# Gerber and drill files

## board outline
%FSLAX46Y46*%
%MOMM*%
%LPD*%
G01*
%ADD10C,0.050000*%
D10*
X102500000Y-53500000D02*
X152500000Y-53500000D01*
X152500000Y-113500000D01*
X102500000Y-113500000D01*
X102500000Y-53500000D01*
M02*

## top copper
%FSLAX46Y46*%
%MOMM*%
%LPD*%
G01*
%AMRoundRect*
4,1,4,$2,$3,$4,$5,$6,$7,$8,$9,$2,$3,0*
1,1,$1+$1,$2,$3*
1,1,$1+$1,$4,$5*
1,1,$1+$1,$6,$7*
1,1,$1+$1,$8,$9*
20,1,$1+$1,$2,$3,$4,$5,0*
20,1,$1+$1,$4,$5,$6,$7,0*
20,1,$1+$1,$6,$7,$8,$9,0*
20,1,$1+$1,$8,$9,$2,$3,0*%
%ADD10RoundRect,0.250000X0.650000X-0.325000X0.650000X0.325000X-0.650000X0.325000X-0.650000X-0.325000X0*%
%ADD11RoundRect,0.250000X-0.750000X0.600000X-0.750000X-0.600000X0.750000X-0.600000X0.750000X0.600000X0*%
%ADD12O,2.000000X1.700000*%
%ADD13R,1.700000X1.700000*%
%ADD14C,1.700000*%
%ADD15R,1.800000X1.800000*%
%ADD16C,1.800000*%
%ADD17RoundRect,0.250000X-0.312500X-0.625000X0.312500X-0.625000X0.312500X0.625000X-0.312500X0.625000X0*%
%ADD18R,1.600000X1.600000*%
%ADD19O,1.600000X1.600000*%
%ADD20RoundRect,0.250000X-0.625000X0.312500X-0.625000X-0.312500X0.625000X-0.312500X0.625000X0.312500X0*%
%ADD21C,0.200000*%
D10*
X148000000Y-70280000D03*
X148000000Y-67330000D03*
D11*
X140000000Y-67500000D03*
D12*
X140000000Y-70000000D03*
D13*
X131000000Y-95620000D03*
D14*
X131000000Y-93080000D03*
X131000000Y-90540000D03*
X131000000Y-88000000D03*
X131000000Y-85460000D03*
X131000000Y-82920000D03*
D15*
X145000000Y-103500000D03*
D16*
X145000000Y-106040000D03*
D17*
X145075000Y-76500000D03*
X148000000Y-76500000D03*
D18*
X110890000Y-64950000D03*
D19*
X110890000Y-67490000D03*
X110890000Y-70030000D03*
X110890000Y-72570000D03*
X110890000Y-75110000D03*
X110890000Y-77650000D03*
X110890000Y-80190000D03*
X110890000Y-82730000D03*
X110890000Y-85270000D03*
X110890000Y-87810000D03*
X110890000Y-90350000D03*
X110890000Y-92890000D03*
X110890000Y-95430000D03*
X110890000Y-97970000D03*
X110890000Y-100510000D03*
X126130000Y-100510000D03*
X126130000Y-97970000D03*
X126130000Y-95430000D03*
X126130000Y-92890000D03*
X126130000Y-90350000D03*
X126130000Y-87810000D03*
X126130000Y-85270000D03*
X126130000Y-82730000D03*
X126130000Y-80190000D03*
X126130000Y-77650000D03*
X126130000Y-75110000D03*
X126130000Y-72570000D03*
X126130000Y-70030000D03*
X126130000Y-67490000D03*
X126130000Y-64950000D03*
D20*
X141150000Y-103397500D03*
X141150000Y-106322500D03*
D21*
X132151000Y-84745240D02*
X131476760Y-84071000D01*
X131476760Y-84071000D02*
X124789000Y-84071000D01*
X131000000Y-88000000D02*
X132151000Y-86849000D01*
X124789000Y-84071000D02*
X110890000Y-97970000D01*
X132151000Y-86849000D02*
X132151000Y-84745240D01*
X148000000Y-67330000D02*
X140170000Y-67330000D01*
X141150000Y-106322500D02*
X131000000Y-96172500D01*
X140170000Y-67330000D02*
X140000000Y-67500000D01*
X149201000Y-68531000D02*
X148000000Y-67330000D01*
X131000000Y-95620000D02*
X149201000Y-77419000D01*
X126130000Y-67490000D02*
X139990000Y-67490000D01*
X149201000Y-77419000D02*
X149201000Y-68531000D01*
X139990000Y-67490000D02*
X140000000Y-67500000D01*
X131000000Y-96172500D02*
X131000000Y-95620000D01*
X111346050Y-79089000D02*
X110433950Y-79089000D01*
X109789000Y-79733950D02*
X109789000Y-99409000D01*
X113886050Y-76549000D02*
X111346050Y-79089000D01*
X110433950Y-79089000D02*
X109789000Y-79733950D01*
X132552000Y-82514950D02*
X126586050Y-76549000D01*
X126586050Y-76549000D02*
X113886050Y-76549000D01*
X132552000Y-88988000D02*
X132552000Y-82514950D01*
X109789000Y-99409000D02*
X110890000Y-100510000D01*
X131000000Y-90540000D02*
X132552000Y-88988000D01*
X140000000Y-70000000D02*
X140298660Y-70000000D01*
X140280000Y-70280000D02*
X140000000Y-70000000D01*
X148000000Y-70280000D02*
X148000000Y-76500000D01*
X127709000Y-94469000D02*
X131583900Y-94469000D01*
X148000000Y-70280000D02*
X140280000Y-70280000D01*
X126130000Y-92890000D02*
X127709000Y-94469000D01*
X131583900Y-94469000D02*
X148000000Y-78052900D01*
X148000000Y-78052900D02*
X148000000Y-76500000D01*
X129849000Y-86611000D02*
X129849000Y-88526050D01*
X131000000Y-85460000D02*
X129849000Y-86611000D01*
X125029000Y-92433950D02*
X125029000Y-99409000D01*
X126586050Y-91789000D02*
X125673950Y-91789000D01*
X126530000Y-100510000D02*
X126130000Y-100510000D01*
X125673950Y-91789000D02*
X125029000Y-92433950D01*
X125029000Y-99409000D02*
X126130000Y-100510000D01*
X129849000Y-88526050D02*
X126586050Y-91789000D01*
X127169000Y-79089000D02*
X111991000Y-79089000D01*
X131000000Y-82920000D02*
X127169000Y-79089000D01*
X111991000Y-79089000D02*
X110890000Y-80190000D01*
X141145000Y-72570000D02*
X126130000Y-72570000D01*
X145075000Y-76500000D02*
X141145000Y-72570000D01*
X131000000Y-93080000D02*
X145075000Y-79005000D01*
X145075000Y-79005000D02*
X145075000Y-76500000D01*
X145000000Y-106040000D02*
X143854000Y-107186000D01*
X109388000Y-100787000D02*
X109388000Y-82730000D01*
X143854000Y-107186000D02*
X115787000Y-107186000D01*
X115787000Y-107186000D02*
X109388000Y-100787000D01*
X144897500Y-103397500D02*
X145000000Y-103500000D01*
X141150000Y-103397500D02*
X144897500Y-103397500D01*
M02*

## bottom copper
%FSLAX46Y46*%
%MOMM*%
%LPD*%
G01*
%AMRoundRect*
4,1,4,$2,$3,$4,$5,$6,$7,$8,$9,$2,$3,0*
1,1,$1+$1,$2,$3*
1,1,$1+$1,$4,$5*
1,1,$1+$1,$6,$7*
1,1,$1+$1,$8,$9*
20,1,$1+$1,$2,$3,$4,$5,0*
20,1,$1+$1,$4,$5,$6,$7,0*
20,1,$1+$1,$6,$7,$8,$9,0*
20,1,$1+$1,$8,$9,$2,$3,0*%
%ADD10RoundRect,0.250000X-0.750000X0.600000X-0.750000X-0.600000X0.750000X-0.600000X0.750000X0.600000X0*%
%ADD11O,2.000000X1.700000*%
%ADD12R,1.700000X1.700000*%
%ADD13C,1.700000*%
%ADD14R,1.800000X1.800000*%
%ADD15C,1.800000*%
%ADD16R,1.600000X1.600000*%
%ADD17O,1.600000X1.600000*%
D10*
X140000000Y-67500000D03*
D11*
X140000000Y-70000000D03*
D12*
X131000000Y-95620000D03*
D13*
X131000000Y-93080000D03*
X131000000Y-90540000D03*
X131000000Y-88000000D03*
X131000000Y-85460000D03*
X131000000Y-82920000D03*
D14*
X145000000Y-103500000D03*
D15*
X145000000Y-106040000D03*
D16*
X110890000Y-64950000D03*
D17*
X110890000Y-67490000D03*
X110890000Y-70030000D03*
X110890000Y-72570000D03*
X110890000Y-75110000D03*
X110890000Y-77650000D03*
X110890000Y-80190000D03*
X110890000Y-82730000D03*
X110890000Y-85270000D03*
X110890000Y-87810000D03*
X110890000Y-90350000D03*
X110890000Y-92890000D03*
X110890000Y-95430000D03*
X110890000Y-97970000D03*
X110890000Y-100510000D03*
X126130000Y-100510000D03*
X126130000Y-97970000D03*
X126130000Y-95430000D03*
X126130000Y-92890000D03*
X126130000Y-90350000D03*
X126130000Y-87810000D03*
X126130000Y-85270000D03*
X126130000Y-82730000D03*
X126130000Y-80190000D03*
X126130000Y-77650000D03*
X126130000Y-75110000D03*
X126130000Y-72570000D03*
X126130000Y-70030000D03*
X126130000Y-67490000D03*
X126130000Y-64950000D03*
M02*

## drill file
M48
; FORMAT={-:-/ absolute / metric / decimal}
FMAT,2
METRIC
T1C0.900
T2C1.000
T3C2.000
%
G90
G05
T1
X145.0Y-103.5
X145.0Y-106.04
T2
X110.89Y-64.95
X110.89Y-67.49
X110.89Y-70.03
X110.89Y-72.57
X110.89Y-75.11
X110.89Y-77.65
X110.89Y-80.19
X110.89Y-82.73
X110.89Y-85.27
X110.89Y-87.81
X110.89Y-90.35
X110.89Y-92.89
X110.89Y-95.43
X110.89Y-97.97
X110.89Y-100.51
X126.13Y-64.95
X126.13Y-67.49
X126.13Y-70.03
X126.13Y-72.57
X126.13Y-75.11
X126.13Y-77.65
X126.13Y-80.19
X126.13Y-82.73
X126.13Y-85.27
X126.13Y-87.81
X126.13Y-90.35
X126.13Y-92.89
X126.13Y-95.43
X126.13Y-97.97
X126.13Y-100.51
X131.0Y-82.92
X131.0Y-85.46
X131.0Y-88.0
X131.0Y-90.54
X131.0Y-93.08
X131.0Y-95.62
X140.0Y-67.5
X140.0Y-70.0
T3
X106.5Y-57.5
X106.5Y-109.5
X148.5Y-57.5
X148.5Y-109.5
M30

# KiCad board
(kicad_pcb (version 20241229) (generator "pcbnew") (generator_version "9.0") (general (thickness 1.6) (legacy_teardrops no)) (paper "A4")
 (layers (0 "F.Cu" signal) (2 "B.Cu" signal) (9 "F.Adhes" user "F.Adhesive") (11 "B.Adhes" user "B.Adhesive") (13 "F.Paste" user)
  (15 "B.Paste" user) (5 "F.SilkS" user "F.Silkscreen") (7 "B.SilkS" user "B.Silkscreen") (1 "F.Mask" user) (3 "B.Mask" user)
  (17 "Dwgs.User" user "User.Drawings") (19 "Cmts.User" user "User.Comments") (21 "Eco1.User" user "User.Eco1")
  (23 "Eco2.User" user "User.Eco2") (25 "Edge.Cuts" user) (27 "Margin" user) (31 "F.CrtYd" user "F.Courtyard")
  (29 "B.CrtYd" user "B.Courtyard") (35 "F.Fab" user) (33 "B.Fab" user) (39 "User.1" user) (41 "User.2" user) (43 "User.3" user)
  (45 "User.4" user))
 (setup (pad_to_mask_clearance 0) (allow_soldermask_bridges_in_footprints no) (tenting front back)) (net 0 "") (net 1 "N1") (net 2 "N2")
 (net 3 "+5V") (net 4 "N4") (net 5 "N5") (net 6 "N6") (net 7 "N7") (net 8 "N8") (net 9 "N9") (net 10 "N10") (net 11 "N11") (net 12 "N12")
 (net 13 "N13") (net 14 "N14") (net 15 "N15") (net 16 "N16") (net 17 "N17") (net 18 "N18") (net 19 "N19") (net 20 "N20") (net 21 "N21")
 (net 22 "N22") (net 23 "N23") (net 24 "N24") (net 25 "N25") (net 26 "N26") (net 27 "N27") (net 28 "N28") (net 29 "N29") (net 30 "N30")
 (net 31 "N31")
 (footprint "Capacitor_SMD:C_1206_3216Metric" (layer "F.Cu") (at 148 68.805 90)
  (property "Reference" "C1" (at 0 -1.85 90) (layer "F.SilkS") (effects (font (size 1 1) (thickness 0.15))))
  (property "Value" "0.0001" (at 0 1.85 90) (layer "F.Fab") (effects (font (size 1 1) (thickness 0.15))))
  (pad "1" smd roundrect (at -1.475 0 90) (size 1.15 1.8) (layers "F.Cu" "F.Mask" "F.Paste") (roundrect_rratio 0.217391) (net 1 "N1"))
  (pad "2" smd roundrect (at 1.475 0 90) (size 1.15 1.8) (layers "F.Cu" "F.Mask" "F.Paste") (roundrect_rratio 0.217391) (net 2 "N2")))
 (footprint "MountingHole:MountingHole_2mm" (layer "F.Cu") (at 148.5 57.5)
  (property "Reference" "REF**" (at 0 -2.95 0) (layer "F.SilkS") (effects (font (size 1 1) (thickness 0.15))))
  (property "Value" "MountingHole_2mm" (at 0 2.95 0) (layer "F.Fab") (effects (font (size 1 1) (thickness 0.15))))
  (pad "" np_thru_hole circle (at 0 0) (size 2 2) (drill 2) (layers "*.Cu" "*.Mask")))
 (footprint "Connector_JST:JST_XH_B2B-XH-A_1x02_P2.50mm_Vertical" (layer "F.Cu") (at 140 67.5 -90)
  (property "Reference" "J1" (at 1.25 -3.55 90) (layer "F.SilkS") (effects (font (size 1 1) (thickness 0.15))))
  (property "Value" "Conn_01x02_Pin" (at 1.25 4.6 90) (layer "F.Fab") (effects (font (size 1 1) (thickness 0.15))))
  (pad "1" thru_hole roundrect (at 0 0 270) (size 1.7 2) (drill 1) (layers "*.Cu" "*.Mask") (remove_unused_layers no)
   (roundrect_rratio 0.147059) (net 2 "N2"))
  (pad "2" thru_hole oval (at 2.5 0 270) (size 1.7 2) (drill 1) (layers "*.Cu" "*.Mask") (remove_unused_layers no) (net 1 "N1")))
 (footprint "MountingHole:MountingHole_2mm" (layer "F.Cu") (at 148.5 109.5)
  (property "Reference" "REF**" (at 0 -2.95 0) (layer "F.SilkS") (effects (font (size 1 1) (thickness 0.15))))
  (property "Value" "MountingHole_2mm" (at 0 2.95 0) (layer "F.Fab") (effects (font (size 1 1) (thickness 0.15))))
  (pad "" np_thru_hole circle (at 0 0) (size 2 2) (drill 2) (layers "*.Cu" "*.Mask")))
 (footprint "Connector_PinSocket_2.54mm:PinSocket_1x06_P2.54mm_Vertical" (layer "F.Cu") (at 131 95.62 180)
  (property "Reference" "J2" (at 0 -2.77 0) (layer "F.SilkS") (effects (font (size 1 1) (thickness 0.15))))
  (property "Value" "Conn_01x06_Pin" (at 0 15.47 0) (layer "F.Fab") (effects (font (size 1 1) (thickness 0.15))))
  (pad "1" thru_hole rect (at 0 0 180) (size 1.7 1.7) (drill 1) (layers "*.Cu" "*.Mask") (remove_unused_layers no) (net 2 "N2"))
  (pad "2" thru_hole circle (at 0 2.54 180) (size 1.7 1.7) (drill 1) (layers "*.Cu" "*.Mask") (remove_unused_layers no) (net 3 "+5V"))
  (pad "3" thru_hole circle (at 0 5.08 180) (size 1.7 1.7) (drill 1) (layers "*.Cu" "*.Mask") (remove_unused_layers no) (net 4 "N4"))
  (pad "4" thru_hole circle (at 0 7.62 180) (size 1.7 1.7) (drill 1) (layers "*.Cu" "*.Mask") (remove_unused_layers no) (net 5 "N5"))
  (pad "5" thru_hole circle (at 0 10.16 180) (size 1.7 1.7) (drill 1) (layers "*.Cu" "*.Mask") (remove_unused_layers no) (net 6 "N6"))
  (pad "6" thru_hole circle (at 0 12.7 180) (size 1.7 1.7) (drill 1) (layers "*.Cu" "*.Mask") (remove_unused_layers no) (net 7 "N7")))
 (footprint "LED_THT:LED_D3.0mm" (layer "F.Cu") (at 145 103.5 -90)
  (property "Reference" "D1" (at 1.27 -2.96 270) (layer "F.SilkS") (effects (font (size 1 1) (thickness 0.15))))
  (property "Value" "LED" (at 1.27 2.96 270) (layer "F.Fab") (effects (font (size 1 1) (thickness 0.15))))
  (pad "1" thru_hole rect (at 0 0 270) (size 1.8 1.8) (drill 0.9) (layers "*.Cu" "*.Mask") (remove_unused_layers no) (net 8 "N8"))
  (pad "2" thru_hole circle (at 2.54 0 270) (size 1.8 1.8) (drill 0.9) (layers "*.Cu" "*.Mask") (remove_unused_layers no) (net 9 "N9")))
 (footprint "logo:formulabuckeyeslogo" (layer "F.Cu") (at 143.014115 88.745726)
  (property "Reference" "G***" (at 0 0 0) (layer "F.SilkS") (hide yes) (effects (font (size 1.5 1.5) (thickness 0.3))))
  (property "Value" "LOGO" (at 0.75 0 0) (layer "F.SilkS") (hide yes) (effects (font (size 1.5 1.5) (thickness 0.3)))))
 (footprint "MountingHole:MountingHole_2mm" (layer "F.Cu") (at 106.5 57.5)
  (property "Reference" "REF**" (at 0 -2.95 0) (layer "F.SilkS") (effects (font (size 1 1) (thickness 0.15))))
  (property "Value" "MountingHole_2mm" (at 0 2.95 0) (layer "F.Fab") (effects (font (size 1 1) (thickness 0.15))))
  (pad "" np_thru_hole circle (at 0 0) (size 2 2) (drill 2) (layers "*.Cu" "*.Mask")))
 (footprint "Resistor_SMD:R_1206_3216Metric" (layer "F.Cu") (at 146.5375 76.5)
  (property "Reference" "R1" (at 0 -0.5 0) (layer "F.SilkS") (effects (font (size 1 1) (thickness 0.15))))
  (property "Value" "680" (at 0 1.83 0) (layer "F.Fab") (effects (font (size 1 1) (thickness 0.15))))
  (pad "1" smd roundrect (at -1.4625 0) (size 1.125 1.75) (layers "F.Cu" "F.Mask" "F.Paste") (roundrect_rratio 0.222222) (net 3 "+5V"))
  (pad "2" smd roundrect (at 1.4625 0) (size 1.125 1.75) (layers "F.Cu" "F.Mask" "F.Paste") (roundrect_rratio 0.222222) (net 1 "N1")))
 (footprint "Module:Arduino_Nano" (layer "F.Cu") (at 110.89 64.95)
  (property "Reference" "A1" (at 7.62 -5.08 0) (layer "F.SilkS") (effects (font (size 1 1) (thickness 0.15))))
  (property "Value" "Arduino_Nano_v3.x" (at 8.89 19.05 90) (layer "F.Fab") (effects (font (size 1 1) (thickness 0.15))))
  (pad "1" thru_hole rect (at 0 0) (size 1.6 1.6) (drill 1) (layers "*.Cu" "*.Mask") (remove_unused_layers no) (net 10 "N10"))
  (pad "2" thru_hole oval (at 0 2.54) (size 1.6 1.6) (drill 1) (layers "*.Cu" "*.Mask") (remove_unused_layers no) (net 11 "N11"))
  (pad "3" thru_hole oval (at 0 5.08) (size 1.6 1.6) (drill 1) (layers "*.Cu" "*.Mask") (remove_unused_layers no) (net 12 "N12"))
  (pad "4" thru_hole oval (at 0 7.62) (size 1.6 1.6) (drill 1) (layers "*.Cu" "*.Mask") (remove_unused_layers no) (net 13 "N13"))
  (pad "5" thru_hole oval (at 0 10.16) (size 1.6 1.6) (drill 1) (layers "*.Cu" "*.Mask") (remove_unused_layers no) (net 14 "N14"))
  (pad "6" thru_hole oval (at 0 12.7) (size 1.6 1.6) (drill 1) (layers "*.Cu" "*.Mask") (remove_unused_layers no) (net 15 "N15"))
  (pad "7" thru_hole oval (at 0 15.24) (size 1.6 1.6) (drill 1) (layers "*.Cu" "*.Mask") (remove_unused_layers no) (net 7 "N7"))
  (pad "8" thru_hole oval (at 0 17.78) (size 1.6 1.6) (drill 1) (layers "*.Cu" "*.Mask") (remove_unused_layers no) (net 9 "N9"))
  (pad "9" thru_hole oval (at 0 20.32) (size 1.6 1.6) (drill 1) (layers "*.Cu" "*.Mask") (remove_unused_layers no) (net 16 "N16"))
  (pad "10" thru_hole oval (at 0 22.86) (size 1.6 1.6) (drill 1) (layers "*.Cu" "*.Mask") (remove_unused_layers no) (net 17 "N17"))
  (pad "11" thru_hole oval (at 0 25.4) (size 1.6 1.6) (drill 1) (layers "*.Cu" "*.Mask") (remove_unused_layers no) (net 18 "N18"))
  (pad "12" thru_hole oval (at 0 27.94) (size 1.6 1.6) (drill 1) (layers "*.Cu" "*.Mask") (remove_unused_layers no) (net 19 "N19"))
  (pad "13" thru_hole oval (at 0 30.48) (size 1.6 1.6) (drill 1) (layers "*.Cu" "*.Mask") (remove_unused_layers no) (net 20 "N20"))
  (pad "14" thru_hole oval (at 0 33.02) (size 1.6 1.6) (drill 1) (layers "*.Cu" "*.Mask") (remove_unused_layers no) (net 5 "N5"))
  (pad "15" thru_hole oval (at 0 35.56) (size 1.6 1.6) (drill 1) (layers "*.Cu" "*.Mask") (remove_unused_layers no) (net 4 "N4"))
  (pad "16" thru_hole oval (at 15.24 35.56) (size 1.6 1.6) (drill 1) (layers "*.Cu" "*.Mask") (remove_unused_layers no) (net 6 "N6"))
  (pad "17" thru_hole oval (at 15.24 33.02) (size 1.6 1.6) (drill 1) (layers "*.Cu" "*.Mask") (remove_unused_layers no) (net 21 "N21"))
  (pad "18" thru_hole oval (at 15.24 30.48) (size 1.6 1.6) (drill 1) (layers "*.Cu" "*.Mask") (remove_unused_layers no) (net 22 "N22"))
  (pad "19" thru_hole oval (at 15.24 27.94) (size 1.6 1.6) (drill 1) (layers "*.Cu" "*.Mask") (remove_unused_layers no) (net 1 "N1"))
  (pad "20" thru_hole oval (at 15.24 25.4) (size 1.6 1.6) (drill 1) (layers "*.Cu" "*.Mask") (remove_unused_layers no) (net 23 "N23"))
  (pad "21" thru_hole oval (at 15.24 22.86) (size 1.6 1.6) (drill 1) (layers "*.Cu" "*.Mask") (remove_unused_layers no) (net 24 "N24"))
  (pad "22" thru_hole oval (at 15.24 20.32) (size 1.6 1.6) (drill 1) (layers "*.Cu" "*.Mask") (remove_unused_layers no) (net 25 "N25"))
  (pad "23" thru_hole oval (at 15.24 17.78) (size 1.6 1.6) (drill 1) (layers "*.Cu" "*.Mask") (remove_unused_layers no) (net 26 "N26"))
  (pad "24" thru_hole oval (at 15.24 15.24) (size 1.6 1.6) (drill 1) (layers "*.Cu" "*.Mask") (remove_unused_layers no) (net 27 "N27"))
  (pad "25" thru_hole oval (at 15.24 12.7) (size 1.6 1.6) (drill 1) (layers "*.Cu" "*.Mask") (remove_unused_layers no) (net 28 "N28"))
  (pad "26" thru_hole oval (at 15.24 10.16) (size 1.6 1.6) (drill 1) (layers "*.Cu" "*.Mask") (remove_unused_layers no) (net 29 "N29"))
  (pad "27" thru_hole oval (at 15.24 7.62) (size 1.6 1.6) (drill 1) (layers "*.Cu" "*.Mask") (remove_unused_layers no) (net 3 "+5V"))
  (pad "28" thru_hole oval (at 15.24 5.08) (size 1.6 1.6) (drill 1) (layers "*.Cu" "*.Mask") (remove_unused_layers no) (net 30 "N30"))
  (pad "29" thru_hole oval (at 15.24 2.54) (size 1.6 1.6) (drill 1) (layers "*.Cu" "*.Mask") (remove_unused_layers no) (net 2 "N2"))
  (pad "30" thru_hole oval (at 15.24 0) (size 1.6 1.6) (drill 1) (layers "*.Cu" "*.Mask") (remove_unused_layers no) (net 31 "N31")))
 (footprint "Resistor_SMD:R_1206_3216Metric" (layer "F.Cu") (at 141.15 104.86 -90)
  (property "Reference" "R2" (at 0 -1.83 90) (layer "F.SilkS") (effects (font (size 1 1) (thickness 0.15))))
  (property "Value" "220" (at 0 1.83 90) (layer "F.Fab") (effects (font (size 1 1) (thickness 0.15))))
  (pad "1" smd roundrect (at -1.4625 0 270) (size 1.125 1.75) (layers "F.Cu" "F.Mask" "F.Paste") (roundrect_rratio 0.222222) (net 8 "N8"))
  (pad "2" smd roundrect (at 1.4625 0 270) (size 1.125 1.75) (layers "F.Cu" "F.Mask" "F.Paste") (roundrect_rratio 0.222222) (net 2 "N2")))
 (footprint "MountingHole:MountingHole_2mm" (layer "F.Cu") (at 106.5 109.5)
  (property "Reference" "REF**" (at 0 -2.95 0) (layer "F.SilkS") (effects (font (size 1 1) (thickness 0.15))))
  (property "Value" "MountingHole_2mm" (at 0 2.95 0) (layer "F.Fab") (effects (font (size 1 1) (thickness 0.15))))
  (pad "" np_thru_hole circle (at 0 0) (size 2 2) (drill 2) (layers "*.Cu" "*.Mask")))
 (gr_rect (start 102.5 53.5) (end 152.5 113.5) (stroke (width 0.05) (type solid)) (fill no) (layer "Edge.Cuts"))
 (segment (start 132.151 84.74524) (end 131.47676 84.071) (width 0.2) (layer "F.Cu") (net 5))
 (segment (start 131.47676 84.071) (end 124.789 84.071) (width 0.2) (layer "F.Cu") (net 5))
 (segment (start 131 88) (end 132.151 86.849) (width 0.2) (layer "F.Cu") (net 5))
 (segment (start 124.789 84.071) (end 110.89 97.97) (width 0.2) (layer "F.Cu") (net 5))
 (segment (start 132.151 86.849) (end 132.151 84.74524) (width 0.2) (layer "F.Cu") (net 5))
 (segment (start 148 67.33) (end 140.17 67.33) (width 0.2) (layer "F.Cu") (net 2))
 (segment (start 141.15 106.3225) (end 131 96.1725) (width 0.2) (layer "F.Cu") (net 2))
 (segment (start 140.17 67.33) (end 140 67.5) (width 0.2) (layer "F.Cu") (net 2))
 (segment (start 149.201 68.531) (end 148 67.33) (width 0.2) (layer "F.Cu") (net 2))
 (segment (start 131 95.62) (end 149.201 77.419) (width 0.2) (layer "F.Cu") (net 2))
 (segment (start 126.13 67.49) (end 139.99 67.49) (width 0.2) (layer "F.Cu") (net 2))
 (segment (start 149.201 77.419) (end 149.201 68.531) (width 0.2) (layer "F.Cu") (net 2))
 (segment (start 139.99 67.49) (end 140 67.5) (width 0.2) (layer "F.Cu") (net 2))
 (segment (start 131 96.1725) (end 131 95.62) (width 0.2) (layer "F.Cu") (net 2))
 (segment (start 111.34605 79.089) (end 110.43395 79.089) (width 0.2) (layer "F.Cu") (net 4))
 (segment (start 109.789 79.73395) (end 109.789 99.409) (width 0.2) (layer "F.Cu") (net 4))
 (segment (start 113.88605 76.549) (end 111.34605 79.089) (width 0.2) (layer "F.Cu") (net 4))
 (segment (start 110.43395 79.089) (end 109.789 79.73395) (width 0.2) (layer "F.Cu") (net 4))
 (segment (start 132.552 82.51495) (end 126.58605 76.549) (width 0.2) (layer "F.Cu") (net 4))
 (segment (start 126.58605 76.549) (end 113.88605 76.549) (width 0.2) (layer "F.Cu") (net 4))
 (segment (start 132.552 88.988) (end 132.552 82.51495) (width 0.2) (layer "F.Cu") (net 4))
 (segment (start 109.789 99.409) (end 110.89 100.51) (width 0.2) (layer "F.Cu") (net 4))
 (segment (start 131 90.54) (end 132.552 88.988) (width 0.2) (layer "F.Cu") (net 4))
 (segment (start 140 70) (end 140.29866 70) (width 0.2) (layer "F.Cu") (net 1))
 (segment (start 140.28 70.28) (end 140 70) (width 0.2) (layer "F.Cu") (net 1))
 (segment (start 148 70.28) (end 148 76.5) (width 0.2) (layer "F.Cu") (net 1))
 (segment (start 127.709 94.469) (end 131.5839 94.469) (width 0.2) (layer "F.Cu") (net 1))
 (segment (start 148 70.28) (end 140.28 70.28) (width 0.2) (layer "F.Cu") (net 1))
 (segment (start 126.13 92.89) (end 127.709 94.469) (width 0.2) (layer "F.Cu") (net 1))
 (segment (start 131.5839 94.469) (end 148 78.0529) (width 0.2) (layer "F.Cu") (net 1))
 (segment (start 148 78.0529) (end 148 76.5) (width 0.2) (layer "F.Cu") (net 1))
 (segment (start 129.849 86.611) (end 129.849 88.52605) (width 0.2) (layer "F.Cu") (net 6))
 (segment (start 131 85.46) (end 129.849 86.611) (width 0.2) (layer "F.Cu") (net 6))
 (segment (start 125.029 92.43395) (end 125.029 99.409) (width 0.2) (layer "F.Cu") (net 6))
 (segment (start 126.58605 91.789) (end 125.67395 91.789) (width 0.2) (layer "F.Cu") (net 6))
 (segment (start 126.53 100.51) (end 126.13 100.51) (width 0.2) (layer "F.Cu") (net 6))
 (segment (start 125.67395 91.789) (end 125.029 92.43395) (width 0.2) (layer "F.Cu") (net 6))
 (segment (start 125.029 99.409) (end 126.13 100.51) (width 0.2) (layer "F.Cu") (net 6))
 (segment (start 129.849 88.52605) (end 126.58605 91.789) (width 0.2) (layer "F.Cu") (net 6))
 (segment (start 127.169 79.089) (end 111.991 79.089) (width 0.2) (layer "F.Cu") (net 7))
 (segment (start 131 82.92) (end 127.169 79.089) (width 0.2) (layer "F.Cu") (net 7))
 (segment (start 111.991 79.089) (end 110.89 80.19) (width 0.2) (layer "F.Cu") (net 7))
 (segment (start 141.145 72.57) (end 126.13 72.57) (width 0.2) (layer "F.Cu") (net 3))
 (segment (start 145.075 76.5) (end 141.145 72.57) (width 0.2) (layer "F.Cu") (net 3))
 (segment (start 131 93.08) (end 145.075 79.005) (width 0.2) (layer "F.Cu") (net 3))
 (segment (start 145.075 79.005) (end 145.075 76.5) (width 0.2) (layer "F.Cu") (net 3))
 (segment (start 145 106.04) (end 143.854 107.186) (width 0.2) (layer "F.Cu") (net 9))
 (segment (start 109.388 100.787) (end 109.388 82.73) (width 0.2) (layer "F.Cu") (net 9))
 (segment (start 143.854 107.186) (end 115.787 107.186) (width 0.2) (layer "F.Cu") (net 9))
 (segment (start 115.787 107.186) (end 109.388 100.787) (width 0.2) (layer "F.Cu") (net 9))
 (segment (start 144.8975 103.3975) (end 145 103.5) (width 0.2) (layer "F.Cu") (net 8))
 (segment (start 141.15 103.3975) (end 144.8975 103.3975) (width 0.2) (layer "F.Cu") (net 8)))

